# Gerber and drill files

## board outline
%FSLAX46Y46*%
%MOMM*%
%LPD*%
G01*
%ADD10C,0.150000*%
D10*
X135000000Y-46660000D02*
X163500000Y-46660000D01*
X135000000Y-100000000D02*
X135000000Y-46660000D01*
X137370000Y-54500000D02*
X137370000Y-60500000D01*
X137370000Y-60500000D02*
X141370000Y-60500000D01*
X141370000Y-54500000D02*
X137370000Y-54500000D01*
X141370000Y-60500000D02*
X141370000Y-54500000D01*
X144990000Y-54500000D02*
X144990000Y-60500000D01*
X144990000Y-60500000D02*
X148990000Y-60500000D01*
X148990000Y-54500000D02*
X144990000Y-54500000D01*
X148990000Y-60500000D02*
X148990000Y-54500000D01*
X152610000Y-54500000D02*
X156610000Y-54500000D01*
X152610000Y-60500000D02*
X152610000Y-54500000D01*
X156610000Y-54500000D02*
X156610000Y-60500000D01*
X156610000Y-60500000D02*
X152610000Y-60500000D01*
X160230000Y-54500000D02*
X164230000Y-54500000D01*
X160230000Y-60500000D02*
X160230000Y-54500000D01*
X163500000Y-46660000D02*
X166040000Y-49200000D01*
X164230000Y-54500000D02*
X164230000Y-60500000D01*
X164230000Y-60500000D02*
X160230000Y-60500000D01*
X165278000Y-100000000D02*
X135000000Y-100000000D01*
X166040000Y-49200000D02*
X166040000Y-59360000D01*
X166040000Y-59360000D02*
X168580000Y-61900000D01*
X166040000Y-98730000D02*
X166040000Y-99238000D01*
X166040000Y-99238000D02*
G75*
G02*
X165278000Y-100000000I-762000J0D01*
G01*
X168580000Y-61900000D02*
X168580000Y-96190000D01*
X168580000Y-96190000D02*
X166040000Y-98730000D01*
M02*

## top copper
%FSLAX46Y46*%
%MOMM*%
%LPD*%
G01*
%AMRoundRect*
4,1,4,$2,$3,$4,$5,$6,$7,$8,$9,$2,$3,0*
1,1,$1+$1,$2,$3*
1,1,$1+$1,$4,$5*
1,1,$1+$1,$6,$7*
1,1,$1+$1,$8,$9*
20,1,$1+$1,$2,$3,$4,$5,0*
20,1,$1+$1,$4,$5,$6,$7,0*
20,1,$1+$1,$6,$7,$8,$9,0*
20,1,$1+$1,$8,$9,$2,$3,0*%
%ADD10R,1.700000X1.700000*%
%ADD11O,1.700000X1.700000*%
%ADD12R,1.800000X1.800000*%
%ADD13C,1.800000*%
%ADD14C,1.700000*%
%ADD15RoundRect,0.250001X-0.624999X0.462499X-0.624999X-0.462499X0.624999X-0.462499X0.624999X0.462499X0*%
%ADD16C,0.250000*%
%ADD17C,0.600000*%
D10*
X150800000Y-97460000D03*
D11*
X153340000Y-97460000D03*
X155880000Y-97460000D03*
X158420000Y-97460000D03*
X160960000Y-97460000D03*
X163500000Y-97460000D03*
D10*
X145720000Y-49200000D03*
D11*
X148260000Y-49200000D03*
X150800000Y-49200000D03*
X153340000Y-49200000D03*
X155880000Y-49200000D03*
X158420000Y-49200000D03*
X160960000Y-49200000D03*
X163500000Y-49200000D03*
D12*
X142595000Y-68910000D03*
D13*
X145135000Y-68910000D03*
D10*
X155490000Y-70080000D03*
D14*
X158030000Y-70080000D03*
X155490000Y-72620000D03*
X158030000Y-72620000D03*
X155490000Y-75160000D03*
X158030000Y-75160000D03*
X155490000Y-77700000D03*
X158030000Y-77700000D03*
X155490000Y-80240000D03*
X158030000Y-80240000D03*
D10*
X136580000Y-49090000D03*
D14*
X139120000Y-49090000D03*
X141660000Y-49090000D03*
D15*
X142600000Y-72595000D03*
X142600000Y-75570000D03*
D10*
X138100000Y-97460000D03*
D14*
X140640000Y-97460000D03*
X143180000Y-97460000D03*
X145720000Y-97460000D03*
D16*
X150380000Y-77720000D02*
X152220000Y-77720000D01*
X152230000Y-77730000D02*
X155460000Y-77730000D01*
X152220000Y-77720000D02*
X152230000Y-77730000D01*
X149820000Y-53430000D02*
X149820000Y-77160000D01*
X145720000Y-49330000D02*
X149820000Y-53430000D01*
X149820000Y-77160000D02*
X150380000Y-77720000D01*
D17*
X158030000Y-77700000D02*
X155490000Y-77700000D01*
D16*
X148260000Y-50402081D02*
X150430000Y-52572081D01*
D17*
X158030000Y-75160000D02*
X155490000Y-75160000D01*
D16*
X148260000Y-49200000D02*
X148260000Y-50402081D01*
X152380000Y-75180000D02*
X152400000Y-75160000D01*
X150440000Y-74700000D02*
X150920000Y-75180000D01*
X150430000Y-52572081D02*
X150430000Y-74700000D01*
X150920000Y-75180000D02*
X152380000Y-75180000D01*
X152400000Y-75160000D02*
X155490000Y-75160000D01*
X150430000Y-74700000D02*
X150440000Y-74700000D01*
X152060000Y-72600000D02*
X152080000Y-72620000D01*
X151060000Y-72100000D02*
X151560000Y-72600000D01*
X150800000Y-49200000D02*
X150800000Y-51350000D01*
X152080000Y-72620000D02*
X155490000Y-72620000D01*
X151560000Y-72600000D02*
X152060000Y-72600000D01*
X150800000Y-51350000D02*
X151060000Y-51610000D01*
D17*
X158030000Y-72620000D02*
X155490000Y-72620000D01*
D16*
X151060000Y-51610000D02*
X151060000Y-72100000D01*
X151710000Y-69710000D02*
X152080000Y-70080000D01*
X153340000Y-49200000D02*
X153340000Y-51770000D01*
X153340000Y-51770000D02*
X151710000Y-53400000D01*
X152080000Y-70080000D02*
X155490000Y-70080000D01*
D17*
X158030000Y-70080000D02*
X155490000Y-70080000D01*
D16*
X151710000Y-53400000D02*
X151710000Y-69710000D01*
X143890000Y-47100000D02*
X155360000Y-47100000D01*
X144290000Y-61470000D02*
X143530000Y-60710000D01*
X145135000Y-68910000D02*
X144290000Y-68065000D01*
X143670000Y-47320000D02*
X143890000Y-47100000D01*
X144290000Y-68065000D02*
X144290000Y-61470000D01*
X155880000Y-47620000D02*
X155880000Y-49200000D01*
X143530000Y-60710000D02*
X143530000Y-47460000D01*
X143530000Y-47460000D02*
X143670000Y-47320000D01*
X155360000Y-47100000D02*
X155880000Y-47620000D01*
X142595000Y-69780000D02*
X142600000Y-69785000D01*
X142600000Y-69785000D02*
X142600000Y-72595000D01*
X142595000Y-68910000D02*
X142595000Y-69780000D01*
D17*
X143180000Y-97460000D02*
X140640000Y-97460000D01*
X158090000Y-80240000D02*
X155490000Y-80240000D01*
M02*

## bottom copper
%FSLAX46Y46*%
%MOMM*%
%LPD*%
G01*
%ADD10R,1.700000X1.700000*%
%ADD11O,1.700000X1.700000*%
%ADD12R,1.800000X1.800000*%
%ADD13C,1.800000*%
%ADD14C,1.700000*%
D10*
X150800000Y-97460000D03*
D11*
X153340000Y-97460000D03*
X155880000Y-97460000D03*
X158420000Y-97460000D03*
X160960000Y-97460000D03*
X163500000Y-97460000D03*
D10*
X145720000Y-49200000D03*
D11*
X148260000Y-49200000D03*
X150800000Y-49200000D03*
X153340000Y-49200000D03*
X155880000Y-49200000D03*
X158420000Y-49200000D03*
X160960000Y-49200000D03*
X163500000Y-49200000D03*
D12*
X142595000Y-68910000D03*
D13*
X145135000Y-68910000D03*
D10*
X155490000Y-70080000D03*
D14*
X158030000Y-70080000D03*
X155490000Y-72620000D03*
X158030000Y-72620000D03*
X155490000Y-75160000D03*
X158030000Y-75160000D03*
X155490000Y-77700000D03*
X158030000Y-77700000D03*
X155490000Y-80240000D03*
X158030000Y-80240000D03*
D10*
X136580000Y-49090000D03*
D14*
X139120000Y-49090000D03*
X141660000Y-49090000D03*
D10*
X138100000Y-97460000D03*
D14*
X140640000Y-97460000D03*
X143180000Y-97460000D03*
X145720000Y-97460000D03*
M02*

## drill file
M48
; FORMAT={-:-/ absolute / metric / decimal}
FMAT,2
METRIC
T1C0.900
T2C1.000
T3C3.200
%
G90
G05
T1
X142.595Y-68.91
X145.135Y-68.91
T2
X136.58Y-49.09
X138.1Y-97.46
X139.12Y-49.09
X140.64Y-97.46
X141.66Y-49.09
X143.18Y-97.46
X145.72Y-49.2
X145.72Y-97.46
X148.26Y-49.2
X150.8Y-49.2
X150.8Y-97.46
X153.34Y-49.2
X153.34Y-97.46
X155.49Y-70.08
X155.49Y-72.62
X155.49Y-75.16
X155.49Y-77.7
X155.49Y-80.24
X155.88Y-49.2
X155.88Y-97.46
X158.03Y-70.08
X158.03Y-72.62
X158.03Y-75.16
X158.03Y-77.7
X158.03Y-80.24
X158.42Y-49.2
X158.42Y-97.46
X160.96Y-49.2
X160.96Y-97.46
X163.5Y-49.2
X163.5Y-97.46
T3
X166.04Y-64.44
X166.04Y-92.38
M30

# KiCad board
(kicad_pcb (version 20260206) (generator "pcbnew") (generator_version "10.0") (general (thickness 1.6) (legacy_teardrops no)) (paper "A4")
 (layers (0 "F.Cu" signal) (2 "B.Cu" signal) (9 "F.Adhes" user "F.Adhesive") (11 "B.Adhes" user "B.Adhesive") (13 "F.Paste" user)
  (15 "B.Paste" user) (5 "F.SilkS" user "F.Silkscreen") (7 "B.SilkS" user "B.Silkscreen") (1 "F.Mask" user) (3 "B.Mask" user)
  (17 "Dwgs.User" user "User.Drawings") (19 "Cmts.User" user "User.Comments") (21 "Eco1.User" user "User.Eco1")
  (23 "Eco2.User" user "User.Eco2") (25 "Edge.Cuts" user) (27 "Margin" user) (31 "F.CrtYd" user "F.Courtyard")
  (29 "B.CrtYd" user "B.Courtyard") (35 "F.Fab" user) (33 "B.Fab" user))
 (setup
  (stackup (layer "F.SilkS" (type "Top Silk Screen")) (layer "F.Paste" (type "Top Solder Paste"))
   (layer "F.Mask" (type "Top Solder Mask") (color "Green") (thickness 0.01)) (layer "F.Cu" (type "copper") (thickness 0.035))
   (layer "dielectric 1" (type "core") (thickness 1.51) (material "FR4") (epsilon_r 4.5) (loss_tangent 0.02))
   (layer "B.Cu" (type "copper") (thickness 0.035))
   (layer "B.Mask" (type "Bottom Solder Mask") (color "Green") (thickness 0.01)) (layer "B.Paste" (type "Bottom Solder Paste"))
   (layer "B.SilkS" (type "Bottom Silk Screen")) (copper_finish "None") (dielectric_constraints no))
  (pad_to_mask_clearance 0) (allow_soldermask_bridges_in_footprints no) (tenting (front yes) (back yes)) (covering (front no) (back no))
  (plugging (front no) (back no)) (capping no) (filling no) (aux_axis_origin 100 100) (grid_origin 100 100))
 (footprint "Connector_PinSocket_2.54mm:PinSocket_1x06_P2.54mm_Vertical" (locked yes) (layer "F.Cu") (at 150.8 97.46 90)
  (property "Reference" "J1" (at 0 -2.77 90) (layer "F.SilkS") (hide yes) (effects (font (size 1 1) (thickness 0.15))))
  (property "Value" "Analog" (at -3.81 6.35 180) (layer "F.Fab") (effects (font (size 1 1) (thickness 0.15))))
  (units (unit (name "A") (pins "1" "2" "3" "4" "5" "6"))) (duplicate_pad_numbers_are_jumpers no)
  (pad "1" thru_hole rect (at 0 0 90) (size 1.7 1.7) (drill 1) (layers "*.Cu" "*.Mask") (remove_unused_layers no) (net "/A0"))
  (pad "2" thru_hole oval (at 0 2.54 90) (size 1.7 1.7) (drill 1) (layers "*.Cu" "*.Mask") (remove_unused_layers no) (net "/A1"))
  (pad "3" thru_hole oval (at 0 5.08 90) (size 1.7 1.7) (drill 1) (layers "*.Cu" "*.Mask") (remove_unused_layers no) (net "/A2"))
  (pad "4" thru_hole oval (at 0 7.62 90) (size 1.7 1.7) (drill 1) (layers "*.Cu" "*.Mask") (remove_unused_layers no) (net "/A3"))
  (pad "5" thru_hole oval (at 0 10.16 90) (size 1.7 1.7) (drill 1) (layers "*.Cu" "*.Mask") (remove_unused_layers no) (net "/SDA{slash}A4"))
  (pad "6" thru_hole oval (at 0 12.7 90) (size 1.7 1.7) (drill 1) (layers "*.Cu" "*.Mask") (remove_unused_layers no) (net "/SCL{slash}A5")))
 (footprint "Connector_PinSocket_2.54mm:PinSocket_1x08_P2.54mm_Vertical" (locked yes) (layer "F.Cu") (at 145.72 49.2 90)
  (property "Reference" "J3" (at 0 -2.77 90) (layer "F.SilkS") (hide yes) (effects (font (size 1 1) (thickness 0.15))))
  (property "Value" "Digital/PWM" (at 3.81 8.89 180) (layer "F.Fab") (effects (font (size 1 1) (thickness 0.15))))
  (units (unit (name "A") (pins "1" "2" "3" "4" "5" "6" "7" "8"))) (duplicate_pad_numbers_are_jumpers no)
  (pad "1" thru_hole rect (at 0 0 90) (size 1.7 1.7) (drill 1) (layers "*.Cu" "*.Mask") (remove_unused_layers no) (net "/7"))
  (pad "2" thru_hole oval (at 0 2.54 90) (size 1.7 1.7) (drill 1) (layers "*.Cu" "*.Mask") (remove_unused_layers no) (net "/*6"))
  (pad "3" thru_hole oval (at 0 5.08 90) (size 1.7 1.7) (drill 1) (layers "*.Cu" "*.Mask") (remove_unused_layers no) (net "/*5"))
  (pad "4" thru_hole oval (at 0 7.62 90) (size 1.7 1.7) (drill 1) (layers "*.Cu" "*.Mask") (remove_unused_layers no) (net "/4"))
  (pad "5" thru_hole oval (at 0 10.16 90) (size 1.7 1.7) (drill 1) (layers "*.Cu" "*.Mask") (remove_unused_layers no) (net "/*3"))
  (pad "6" thru_hole oval (at 0 12.7 90) (size 1.7 1.7) (drill 1) (layers "*.Cu" "*.Mask") (remove_unused_layers no) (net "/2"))
  (pad "7" thru_hole oval (at 0 15.24 90) (size 1.7 1.7) (drill 1) (layers "*.Cu" "*.Mask") (remove_unused_layers no) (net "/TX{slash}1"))
  (pad "8" thru_hole oval (at 0 17.78 90) (size 1.7 1.7) (drill 1) (layers "*.Cu" "*.Mask") (remove_unused_layers no) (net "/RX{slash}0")))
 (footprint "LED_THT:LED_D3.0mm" (layer "F.Cu") (at 142.595 68.91)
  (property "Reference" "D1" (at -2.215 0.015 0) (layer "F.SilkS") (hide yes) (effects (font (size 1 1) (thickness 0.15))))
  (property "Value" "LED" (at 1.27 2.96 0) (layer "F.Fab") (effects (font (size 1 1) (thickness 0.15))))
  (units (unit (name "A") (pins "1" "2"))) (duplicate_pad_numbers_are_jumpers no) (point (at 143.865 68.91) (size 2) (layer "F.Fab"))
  (pad "1" thru_hole rect (at 0 0) (size 1.8 1.8) (drill 0.9) (layers "*.Cu" "*.Mask") (remove_unused_layers no) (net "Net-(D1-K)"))
  (pad "2" thru_hole circle (at 2.54 0) (size 1.8 1.8) (drill 0.9) (layers "*.Cu" "*.Mask") (remove_unused_layers no) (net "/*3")))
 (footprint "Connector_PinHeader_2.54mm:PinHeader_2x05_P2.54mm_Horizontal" (layer "F.Cu") (at 155.49 70.08)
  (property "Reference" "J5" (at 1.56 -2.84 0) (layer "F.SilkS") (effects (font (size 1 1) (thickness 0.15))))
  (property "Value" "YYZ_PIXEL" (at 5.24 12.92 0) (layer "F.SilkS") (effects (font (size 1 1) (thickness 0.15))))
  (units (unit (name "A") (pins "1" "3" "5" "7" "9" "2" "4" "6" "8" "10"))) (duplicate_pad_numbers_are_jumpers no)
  (pad "1" thru_hole rect (at 0 0) (size 1.7 1.7) (drill 1) (layers "*.Cu" "*.Mask") (remove_unused_layers no) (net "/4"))
  (pad "2" thru_hole circle (at 2.54 0) (size 1.7 1.7) (drill 1) (layers "*.Cu" "*.Mask") (remove_unused_layers no) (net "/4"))
  (pad "3" thru_hole circle (at 0 2.54) (size 1.7 1.7) (drill 1) (layers "*.Cu" "*.Mask") (remove_unused_layers no) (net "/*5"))
  (pad "4" thru_hole circle (at 2.54 2.54) (size 1.7 1.7) (drill 1) (layers "*.Cu" "*.Mask") (remove_unused_layers no) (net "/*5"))
  (pad "5" thru_hole circle (at 0 5.08) (size 1.7 1.7) (drill 1) (layers "*.Cu" "*.Mask") (remove_unused_layers no) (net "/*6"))
  (pad "6" thru_hole circle (at 2.54 5.08) (size 1.7 1.7) (drill 1) (layers "*.Cu" "*.Mask") (remove_unused_layers no) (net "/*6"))
  (pad "7" thru_hole circle (at 0 7.62) (size 1.7 1.7) (drill 1) (layers "*.Cu" "*.Mask") (remove_unused_layers no) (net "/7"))
  (pad "8" thru_hole circle (at 2.54 7.62) (size 1.7 1.7) (drill 1) (layers "*.Cu" "*.Mask") (remove_unused_layers no) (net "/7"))
  (pad "9" thru_hole circle (at 0 10.16) (size 1.7 1.7) (drill 1) (layers "*.Cu" "*.Mask") (remove_unused_layers no) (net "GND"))
  (pad "10" thru_hole circle (at 2.54 10.16) (size 1.7 1.7) (drill 1) (layers "*.Cu" "*.Mask") (remove_unused_layers no) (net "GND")))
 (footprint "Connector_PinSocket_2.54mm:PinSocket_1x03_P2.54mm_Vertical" (layer "F.Cu") (at 136.58 49.09 90)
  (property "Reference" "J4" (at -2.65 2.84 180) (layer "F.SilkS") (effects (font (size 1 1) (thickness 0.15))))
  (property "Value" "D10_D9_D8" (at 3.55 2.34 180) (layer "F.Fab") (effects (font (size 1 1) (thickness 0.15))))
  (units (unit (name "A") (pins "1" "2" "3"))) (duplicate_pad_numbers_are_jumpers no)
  (pad "1" thru_hole rect (at 0 0 90) (size 1.7 1.7) (drill 1) (layers "*.Cu" "*.Mask") (remove_unused_layers no)
   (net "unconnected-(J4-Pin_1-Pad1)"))
  (pad "2" thru_hole circle (at 0 2.54 90) (size 1.7 1.7) (drill 1) (layers "*.Cu" "*.Mask") (remove_unused_layers no)
   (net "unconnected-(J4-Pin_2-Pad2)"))
  (pad "3" thru_hole circle (at 0 5.08 90) (size 1.7 1.7) (drill 1) (layers "*.Cu" "*.Mask") (remove_unused_layers no)
   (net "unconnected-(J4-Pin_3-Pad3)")))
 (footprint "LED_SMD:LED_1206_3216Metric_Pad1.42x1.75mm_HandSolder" (layer "F.Cu") (at 142.6 74.0825 -90)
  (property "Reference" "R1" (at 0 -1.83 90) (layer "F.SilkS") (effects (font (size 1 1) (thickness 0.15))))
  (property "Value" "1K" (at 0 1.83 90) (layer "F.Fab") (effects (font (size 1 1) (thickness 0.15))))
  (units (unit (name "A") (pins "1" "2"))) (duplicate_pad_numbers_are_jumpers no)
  (pad "1" smd roundrect (at -1.4875 0 270) (size 1.425 1.75) (layers "F.Cu" "F.Mask" "F.Paste") (roundrect_rratio 0.175439)
   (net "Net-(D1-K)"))
  (pad "2" smd roundrect (at 1.4875 0 270) (size 1.425 1.75) (layers "F.Cu" "F.Mask" "F.Paste") (roundrect_rratio 0.175439) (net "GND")))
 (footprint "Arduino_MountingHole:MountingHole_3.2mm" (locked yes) (layer "F.Cu") (at 166.04 64.44)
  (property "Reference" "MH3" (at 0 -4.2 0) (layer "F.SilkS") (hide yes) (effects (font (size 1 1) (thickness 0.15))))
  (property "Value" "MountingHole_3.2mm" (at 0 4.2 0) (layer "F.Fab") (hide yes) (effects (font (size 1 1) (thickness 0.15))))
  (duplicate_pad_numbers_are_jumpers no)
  (pad "" np_thru_hole circle (at 0 0) (size 3.2 3.2) (drill 3.2) (layers "*.Cu" "*.Mask")))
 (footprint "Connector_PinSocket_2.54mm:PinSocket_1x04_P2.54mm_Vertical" (layer "F.Cu") (at 138.1 97.46 90)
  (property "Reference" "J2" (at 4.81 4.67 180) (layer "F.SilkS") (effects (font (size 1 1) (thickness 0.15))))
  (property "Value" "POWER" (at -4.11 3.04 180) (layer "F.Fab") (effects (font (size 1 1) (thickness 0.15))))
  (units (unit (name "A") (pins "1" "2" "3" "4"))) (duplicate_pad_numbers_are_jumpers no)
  (pad "1" thru_hole rect (at 0 0 90) (size 1.7 1.7) (drill 1) (layers "*.Cu" "*.Mask") (remove_unused_layers no) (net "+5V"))
  (pad "2" thru_hole circle (at 0 2.54 90) (size 1.7 1.7) (drill 1) (layers "*.Cu" "*.Mask") (remove_unused_layers no) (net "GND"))
  (pad "3" thru_hole circle (at 0 5.08 90) (size 1.7 1.7) (drill 1) (layers "*.Cu" "*.Mask") (remove_unused_layers no) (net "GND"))
  (pad "4" thru_hole circle (at 0 7.62 90) (size 1.7 1.7) (drill 1) (layers "*.Cu" "*.Mask") (remove_unused_layers no) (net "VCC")))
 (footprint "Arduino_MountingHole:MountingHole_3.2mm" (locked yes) (layer "F.Cu") (at 166.04 92.38)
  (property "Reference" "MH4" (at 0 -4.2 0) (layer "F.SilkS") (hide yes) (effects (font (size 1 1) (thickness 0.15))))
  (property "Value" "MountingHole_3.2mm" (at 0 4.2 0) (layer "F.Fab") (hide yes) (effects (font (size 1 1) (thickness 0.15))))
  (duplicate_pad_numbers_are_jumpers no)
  (pad "" np_thru_hole circle (at 0 0) (size 3.2 3.2) (drill 3.2) (layers "*.Cu" "*.Mask")))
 (gr_line (start 135 46.66) (end 163.5 46.66) (stroke (width 0.15) (type solid)) (layer "Edge.Cuts"))
 (gr_line (start 135 100) (end 135 46.66) (stroke (width 0.15) (type solid)) (layer "Edge.Cuts"))
 (gr_line (start 137.37 54.5) (end 137.37 60.5) (stroke (width 0.15) (type solid)) (layer "Edge.Cuts"))
 (gr_line (start 137.37 60.5) (end 141.37 60.5) (stroke (width 0.15) (type solid)) (layer "Edge.Cuts"))
 (gr_line (start 141.37 54.5) (end 137.37 54.5) (stroke (width 0.15) (type solid)) (layer "Edge.Cuts"))
 (gr_line (start 141.37 60.5) (end 141.37 54.5) (stroke (width 0.15) (type solid)) (layer "Edge.Cuts"))
 (gr_line (start 144.99 54.5) (end 144.99 60.5) (stroke (width 0.15) (type default)) (layer "Edge.Cuts"))
 (gr_line (start 144.99 60.5) (end 148.99 60.5) (stroke (width 0.15) (type default)) (layer "Edge.Cuts"))
 (gr_line (start 148.99 54.5) (end 144.99 54.5) (stroke (width 0.15) (type default)) (layer "Edge.Cuts"))
 (gr_line (start 148.99 60.5) (end 148.99 54.5) (stroke (width 0.15) (type default)) (layer "Edge.Cuts"))
 (gr_line (start 152.61 54.5) (end 156.61 54.5) (stroke (width 0.15) (type solid)) (layer "Edge.Cuts"))
 (gr_line (start 152.61 60.5) (end 152.61 54.5) (stroke (width 0.15) (type solid)) (layer "Edge.Cuts"))
 (gr_line (start 156.61 54.5) (end 156.61 60.5) (stroke (width 0.15) (type solid)) (layer "Edge.Cuts"))
 (gr_line (start 156.61 60.5) (end 152.61 60.5) (stroke (width 0.15) (type solid)) (layer "Edge.Cuts"))
 (gr_line (start 160.23 54.5) (end 164.23 54.5) (stroke (width 0.15) (type solid)) (layer "Edge.Cuts"))
 (gr_line (start 160.23 60.5) (end 160.23 54.5) (stroke (width 0.15) (type solid)) (layer "Edge.Cuts"))
 (gr_line (start 163.5 46.66) (end 166.04 49.2) (stroke (width 0.15) (type solid)) (layer "Edge.Cuts"))
 (gr_line (start 164.23 54.5) (end 164.23 60.5) (stroke (width 0.15) (type solid)) (layer "Edge.Cuts"))
 (gr_line (start 164.23 60.5) (end 160.23 60.5) (stroke (width 0.15) (type solid)) (layer "Edge.Cuts"))
 (gr_line (start 165.278 100) (end 135 100) (stroke (width 0.15) (type solid)) (layer "Edge.Cuts"))
 (gr_line (start 166.04 49.2) (end 166.04 59.36) (stroke (width 0.15) (type solid)) (layer "Edge.Cuts"))
 (gr_line (start 166.04 59.36) (end 168.58 61.9) (stroke (width 0.15) (type solid)) (layer "Edge.Cuts"))
 (gr_line (start 166.04 98.73) (end 166.04 99.238) (stroke (width 0.15) (type solid)) (layer "Edge.Cuts"))
 (gr_arc (start 166.04 99.238) (mid 165.816815 99.776815) (end 165.278 100) (stroke (width 0.15) (type solid)) (layer "Edge.Cuts"))
 (gr_line (start 168.58 61.9) (end 168.58 96.19) (stroke (width 0.15) (type solid)) (layer "Edge.Cuts"))
 (gr_line (start 168.58 96.19) (end 166.04 98.73) (stroke (width 0.15) (type solid)) (layer "Edge.Cuts"))
 (segment (start 150.38 77.72) (end 152.22 77.72) (width 0.25) (layer "F.Cu") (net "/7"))
 (segment (start 152.23 77.73) (end 155.46 77.73) (width 0.25) (layer "F.Cu") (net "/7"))
 (segment (start 152.22 77.72) (end 152.23 77.73) (width 0.25) (layer "F.Cu") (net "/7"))
 (segment (start 149.82 53.43) (end 149.82 77.16) (width 0.25) (layer "F.Cu") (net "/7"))
 (segment (start 145.72 49.33) (end 149.82 53.43) (width 0.25) (layer "F.Cu") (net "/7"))
 (segment (start 149.82 77.16) (end 150.38 77.72) (width 0.25) (layer "F.Cu") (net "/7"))
 (segment (start 158.03 77.7) (end 155.49 77.7) (width 0.6) (layer "F.Cu") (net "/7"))
 (segment (start 148.26 50.402081) (end 150.43 52.572081) (width 0.25) (layer "F.Cu") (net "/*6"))
 (segment (start 158.03 75.16) (end 155.49 75.16) (width 0.6) (layer "F.Cu") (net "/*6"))
 (segment (start 148.26 49.2) (end 148.26 50.402081) (width 0.25) (layer "F.Cu") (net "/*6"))
 (segment (start 152.38 75.18) (end 152.4 75.16) (width 0.25) (layer "F.Cu") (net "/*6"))
 (segment (start 150.44 74.7) (end 150.92 75.18) (width 0.25) (layer "F.Cu") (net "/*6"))
 (segment (start 150.43 52.572081) (end 150.43 74.7) (width 0.25) (layer "F.Cu") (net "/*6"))
 (segment (start 150.92 75.18) (end 152.38 75.18) (width 0.25) (layer "F.Cu") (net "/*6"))
 (segment (start 152.4 75.16) (end 155.49 75.16) (width 0.25) (layer "F.Cu") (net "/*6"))
 (segment (start 150.43 74.7) (end 150.44 74.7) (width 0.25) (layer "F.Cu") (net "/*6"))
 (segment (start 152.06 72.6) (end 152.08 72.62) (width 0.25) (layer "F.Cu") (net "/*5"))
 (segment (start 151.06 72.1) (end 151.56 72.6) (width 0.25) (layer "F.Cu") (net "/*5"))
 (segment (start 150.8 49.2) (end 150.8 51.35) (width 0.25) (layer "F.Cu") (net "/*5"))
 (segment (start 152.08 72.62) (end 155.49 72.62) (width 0.25) (layer "F.Cu") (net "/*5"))
 (segment (start 151.56 72.6) (end 152.06 72.6) (width 0.25) (layer "F.Cu") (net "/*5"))
 (segment (start 150.8 51.35) (end 151.06 51.61) (width 0.25) (layer "F.Cu") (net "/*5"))
 (segment (start 158.03 72.62) (end 155.49 72.62) (width 0.6) (layer "F.Cu") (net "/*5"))
 (segment (start 151.06 51.61) (end 151.06 72.1) (width 0.25) (layer "F.Cu") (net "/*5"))
 (segment (start 151.71 69.71) (end 152.08 70.08) (width 0.25) (layer "F.Cu") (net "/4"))
 (segment (start 153.34 49.2) (end 153.34 51.77) (width 0.25) (layer "F.Cu") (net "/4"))
 (segment (start 153.34 51.77) (end 151.71 53.4) (width 0.25) (layer "F.Cu") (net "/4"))
 (segment (start 152.08 70.08) (end 155.49 70.08) (width 0.25) (layer "F.Cu") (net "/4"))
 (segment (start 158.03 70.08) (end 155.49 70.08) (width 0.6) (layer "F.Cu") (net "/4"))
 (segment (start 151.71 53.4) (end 151.71 69.71) (width 0.25) (layer "F.Cu") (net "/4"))
 (segment (start 143.89 47.1) (end 155.36 47.1) (width 0.25) (layer "F.Cu") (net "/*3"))
 (segment (start 144.29 61.47) (end 143.53 60.71) (width 0.25) (layer "F.Cu") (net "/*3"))
 (segment (start 145.135 68.91) (end 144.29 68.065) (width 0.25) (layer "F.Cu") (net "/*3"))
 (segment (start 143.67 47.32) (end 143.89 47.1) (width 0.25) (layer "F.Cu") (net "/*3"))
 (segment (start 144.29 68.065) (end 144.29 61.47) (width 0.25) (layer "F.Cu") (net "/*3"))
 (segment (start 155.88 47.62) (end 155.88 49.2) (width 0.25) (layer "F.Cu") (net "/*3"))
 (segment (start 143.53 60.71) (end 143.53 47.46) (width 0.25) (layer "F.Cu") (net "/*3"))
 (segment (start 143.53 47.46) (end 143.67 47.32) (width 0.25) (layer "F.Cu") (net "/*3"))
 (segment (start 155.36 47.1) (end 155.88 47.62) (width 0.25) (layer "F.Cu") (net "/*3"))
 (segment (start 142.595 69.78) (end 142.6 69.785) (width 0.25) (layer "F.Cu") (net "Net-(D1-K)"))
 (segment (start 142.6 69.785) (end 142.6 72.595) (width 0.25) (layer "F.Cu") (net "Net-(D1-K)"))
 (segment (start 142.595 68.91) (end 142.595 69.78) (width 0.25) (layer "F.Cu") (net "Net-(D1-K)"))
 (segment (start 143.18 97.46) (end 140.64 97.46) (width 0.6) (layer "F.Cu") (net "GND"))
 (segment (start 158.09 80.24) (end 155.49 80.24) (width 0.6) (layer "F.Cu") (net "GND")))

